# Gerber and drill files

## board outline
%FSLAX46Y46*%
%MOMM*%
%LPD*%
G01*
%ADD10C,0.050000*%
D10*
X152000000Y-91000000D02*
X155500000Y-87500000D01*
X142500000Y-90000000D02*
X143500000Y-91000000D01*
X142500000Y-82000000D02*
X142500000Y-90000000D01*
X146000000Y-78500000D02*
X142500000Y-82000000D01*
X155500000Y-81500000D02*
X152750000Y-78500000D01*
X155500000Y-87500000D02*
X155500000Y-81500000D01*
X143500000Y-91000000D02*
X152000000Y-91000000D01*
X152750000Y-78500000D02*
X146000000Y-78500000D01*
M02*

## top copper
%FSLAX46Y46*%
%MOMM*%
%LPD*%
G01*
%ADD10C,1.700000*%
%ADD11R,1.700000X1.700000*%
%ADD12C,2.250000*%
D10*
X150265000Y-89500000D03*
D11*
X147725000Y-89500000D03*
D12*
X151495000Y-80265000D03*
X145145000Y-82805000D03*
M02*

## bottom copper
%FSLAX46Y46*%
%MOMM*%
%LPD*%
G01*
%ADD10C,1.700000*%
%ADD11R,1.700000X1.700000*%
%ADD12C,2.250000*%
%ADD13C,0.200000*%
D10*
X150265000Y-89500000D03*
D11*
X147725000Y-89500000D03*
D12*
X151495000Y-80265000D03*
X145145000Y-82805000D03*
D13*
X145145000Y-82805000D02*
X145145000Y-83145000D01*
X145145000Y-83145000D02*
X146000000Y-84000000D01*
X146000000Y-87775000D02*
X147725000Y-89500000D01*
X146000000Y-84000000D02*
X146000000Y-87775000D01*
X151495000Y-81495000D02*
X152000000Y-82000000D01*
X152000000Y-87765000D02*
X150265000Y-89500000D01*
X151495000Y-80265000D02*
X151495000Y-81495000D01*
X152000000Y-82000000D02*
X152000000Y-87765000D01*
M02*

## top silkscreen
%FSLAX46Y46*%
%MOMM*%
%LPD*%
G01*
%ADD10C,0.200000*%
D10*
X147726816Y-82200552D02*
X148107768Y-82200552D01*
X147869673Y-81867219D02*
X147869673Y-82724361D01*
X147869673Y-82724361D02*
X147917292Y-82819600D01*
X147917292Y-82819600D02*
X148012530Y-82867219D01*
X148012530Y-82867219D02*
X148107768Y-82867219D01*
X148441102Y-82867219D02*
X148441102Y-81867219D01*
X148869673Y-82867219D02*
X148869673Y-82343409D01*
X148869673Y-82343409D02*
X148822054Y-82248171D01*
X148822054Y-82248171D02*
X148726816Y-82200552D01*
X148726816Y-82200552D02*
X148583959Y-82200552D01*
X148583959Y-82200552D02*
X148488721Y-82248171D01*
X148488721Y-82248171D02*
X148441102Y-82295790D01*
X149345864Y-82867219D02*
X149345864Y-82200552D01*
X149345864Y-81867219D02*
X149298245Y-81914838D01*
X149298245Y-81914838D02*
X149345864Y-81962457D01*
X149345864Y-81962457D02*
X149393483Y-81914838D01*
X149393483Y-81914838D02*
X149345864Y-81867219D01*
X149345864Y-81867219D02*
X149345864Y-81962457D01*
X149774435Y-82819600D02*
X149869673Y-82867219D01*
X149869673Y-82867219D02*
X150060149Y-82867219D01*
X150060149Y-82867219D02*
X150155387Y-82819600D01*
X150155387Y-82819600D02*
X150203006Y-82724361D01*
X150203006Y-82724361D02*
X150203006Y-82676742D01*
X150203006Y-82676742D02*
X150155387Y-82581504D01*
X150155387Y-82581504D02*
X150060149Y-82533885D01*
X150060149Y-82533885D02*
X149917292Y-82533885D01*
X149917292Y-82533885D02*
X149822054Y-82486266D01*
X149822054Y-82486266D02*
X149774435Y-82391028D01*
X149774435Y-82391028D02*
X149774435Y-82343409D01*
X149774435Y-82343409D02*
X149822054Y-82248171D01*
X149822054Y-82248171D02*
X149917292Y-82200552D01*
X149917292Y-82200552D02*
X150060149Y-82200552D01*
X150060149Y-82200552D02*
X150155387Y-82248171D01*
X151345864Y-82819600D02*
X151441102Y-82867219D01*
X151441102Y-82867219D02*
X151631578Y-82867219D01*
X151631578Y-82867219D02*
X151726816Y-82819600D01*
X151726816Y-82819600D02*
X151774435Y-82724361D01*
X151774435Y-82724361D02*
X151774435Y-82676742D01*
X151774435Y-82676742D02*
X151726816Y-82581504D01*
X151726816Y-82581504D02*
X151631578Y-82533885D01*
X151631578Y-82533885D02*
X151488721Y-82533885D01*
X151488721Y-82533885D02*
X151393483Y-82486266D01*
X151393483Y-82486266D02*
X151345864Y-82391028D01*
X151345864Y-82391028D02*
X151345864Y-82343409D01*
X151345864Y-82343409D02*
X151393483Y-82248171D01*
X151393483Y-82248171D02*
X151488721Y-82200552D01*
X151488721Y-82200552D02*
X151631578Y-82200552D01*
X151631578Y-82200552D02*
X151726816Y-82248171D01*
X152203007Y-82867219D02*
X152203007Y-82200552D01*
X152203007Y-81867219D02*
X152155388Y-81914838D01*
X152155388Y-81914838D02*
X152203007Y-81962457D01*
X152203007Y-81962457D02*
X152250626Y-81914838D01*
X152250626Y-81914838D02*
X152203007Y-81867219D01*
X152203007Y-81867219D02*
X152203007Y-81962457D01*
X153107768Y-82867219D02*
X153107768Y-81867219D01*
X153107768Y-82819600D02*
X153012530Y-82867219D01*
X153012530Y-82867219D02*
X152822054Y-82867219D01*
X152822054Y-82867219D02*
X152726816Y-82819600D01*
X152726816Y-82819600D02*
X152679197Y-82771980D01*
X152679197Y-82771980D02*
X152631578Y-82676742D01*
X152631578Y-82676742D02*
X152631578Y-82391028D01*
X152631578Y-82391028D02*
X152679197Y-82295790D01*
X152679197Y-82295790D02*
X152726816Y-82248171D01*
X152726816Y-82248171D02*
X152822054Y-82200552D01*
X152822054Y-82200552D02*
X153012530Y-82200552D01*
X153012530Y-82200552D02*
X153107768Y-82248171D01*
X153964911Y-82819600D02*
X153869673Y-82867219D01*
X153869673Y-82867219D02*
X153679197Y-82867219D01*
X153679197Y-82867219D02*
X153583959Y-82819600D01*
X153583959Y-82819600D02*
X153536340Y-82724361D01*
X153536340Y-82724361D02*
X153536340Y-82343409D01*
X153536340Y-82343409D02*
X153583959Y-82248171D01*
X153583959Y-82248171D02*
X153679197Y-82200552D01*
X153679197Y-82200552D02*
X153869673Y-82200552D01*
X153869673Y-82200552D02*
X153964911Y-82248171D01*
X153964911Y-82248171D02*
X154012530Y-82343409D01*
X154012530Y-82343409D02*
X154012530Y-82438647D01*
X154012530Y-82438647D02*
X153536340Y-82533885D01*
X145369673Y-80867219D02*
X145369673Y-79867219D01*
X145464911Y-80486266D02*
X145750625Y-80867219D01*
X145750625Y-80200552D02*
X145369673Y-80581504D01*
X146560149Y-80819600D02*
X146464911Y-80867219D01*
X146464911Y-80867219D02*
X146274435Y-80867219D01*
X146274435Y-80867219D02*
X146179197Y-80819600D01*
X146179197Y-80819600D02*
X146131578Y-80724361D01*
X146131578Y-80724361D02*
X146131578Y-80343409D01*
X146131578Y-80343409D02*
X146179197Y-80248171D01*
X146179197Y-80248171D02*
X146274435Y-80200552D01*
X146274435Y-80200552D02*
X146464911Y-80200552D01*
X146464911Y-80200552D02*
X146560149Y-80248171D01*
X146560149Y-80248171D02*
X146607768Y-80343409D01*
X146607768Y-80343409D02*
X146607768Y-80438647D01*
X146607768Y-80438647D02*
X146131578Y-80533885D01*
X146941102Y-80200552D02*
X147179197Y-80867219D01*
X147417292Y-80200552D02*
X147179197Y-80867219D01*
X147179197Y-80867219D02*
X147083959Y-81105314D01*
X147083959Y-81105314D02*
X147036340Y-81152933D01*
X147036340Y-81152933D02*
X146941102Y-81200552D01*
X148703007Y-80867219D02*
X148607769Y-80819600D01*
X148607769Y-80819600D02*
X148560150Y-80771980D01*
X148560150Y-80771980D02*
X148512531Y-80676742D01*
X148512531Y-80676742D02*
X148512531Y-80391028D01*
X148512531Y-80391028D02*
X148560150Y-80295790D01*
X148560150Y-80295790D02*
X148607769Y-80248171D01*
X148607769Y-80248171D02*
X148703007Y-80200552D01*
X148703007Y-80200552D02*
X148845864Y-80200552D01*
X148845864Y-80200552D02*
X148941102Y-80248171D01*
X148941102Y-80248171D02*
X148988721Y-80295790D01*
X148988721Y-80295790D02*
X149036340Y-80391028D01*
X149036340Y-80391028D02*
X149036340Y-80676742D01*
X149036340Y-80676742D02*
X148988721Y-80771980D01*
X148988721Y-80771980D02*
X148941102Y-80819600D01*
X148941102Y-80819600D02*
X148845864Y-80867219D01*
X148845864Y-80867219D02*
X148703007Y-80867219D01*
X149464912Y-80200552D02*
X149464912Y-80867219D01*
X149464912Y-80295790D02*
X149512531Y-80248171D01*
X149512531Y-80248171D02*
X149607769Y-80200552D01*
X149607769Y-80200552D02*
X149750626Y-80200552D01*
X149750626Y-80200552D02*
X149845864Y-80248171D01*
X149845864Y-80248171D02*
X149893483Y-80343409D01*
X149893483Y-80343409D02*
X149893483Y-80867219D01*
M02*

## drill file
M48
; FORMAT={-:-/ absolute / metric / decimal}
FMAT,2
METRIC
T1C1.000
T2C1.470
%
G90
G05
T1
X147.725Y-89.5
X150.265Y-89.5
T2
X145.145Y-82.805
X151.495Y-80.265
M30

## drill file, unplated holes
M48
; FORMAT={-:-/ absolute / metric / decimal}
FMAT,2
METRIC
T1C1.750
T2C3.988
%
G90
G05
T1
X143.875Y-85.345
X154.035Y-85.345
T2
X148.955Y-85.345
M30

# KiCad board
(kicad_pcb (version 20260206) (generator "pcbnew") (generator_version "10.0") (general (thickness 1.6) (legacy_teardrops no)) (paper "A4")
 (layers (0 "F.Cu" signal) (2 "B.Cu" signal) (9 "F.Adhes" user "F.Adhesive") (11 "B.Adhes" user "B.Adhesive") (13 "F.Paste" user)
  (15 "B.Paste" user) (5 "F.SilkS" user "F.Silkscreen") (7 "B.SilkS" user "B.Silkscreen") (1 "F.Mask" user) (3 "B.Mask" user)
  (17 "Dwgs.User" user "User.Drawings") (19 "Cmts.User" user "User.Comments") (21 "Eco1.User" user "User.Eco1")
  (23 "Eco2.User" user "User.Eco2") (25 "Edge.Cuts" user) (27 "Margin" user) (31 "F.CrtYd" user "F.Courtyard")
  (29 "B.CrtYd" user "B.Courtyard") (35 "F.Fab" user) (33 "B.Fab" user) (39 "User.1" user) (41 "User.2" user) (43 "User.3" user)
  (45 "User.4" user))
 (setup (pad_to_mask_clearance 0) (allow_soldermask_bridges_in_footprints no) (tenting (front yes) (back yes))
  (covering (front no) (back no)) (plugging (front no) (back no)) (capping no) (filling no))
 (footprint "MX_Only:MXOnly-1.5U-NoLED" (layer "F.Cu") (at 148.955 85.345)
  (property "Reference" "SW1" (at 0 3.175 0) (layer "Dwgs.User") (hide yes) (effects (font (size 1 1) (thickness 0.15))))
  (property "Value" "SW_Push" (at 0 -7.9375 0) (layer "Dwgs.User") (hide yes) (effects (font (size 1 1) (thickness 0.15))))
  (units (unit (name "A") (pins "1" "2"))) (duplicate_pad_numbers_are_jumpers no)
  (pad "" np_thru_hole circle (at -5.08 0 48.0996) (size 1.75 1.75) (drill 1.75) (layers "*.Cu" "*.Mask"))
  (pad "" np_thru_hole circle (at 0 0) (size 3.9878 3.9878) (drill 3.9878) (layers "*.Cu" "*.Mask"))
  (pad "" np_thru_hole circle (at 5.08 0 48.0996) (size 1.75 1.75) (drill 1.75) (layers "*.Cu" "*.Mask"))
  (pad "1" thru_hole circle (at -3.81 -2.54) (size 2.25 2.25) (drill 1.47) (layers "*.Cu" "B.Mask") (remove_unused_layers no)
   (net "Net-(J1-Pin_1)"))
  (pad "2" thru_hole circle (at 2.54 -5.08) (size 2.25 2.25) (drill 1.47) (layers "*.Cu" "B.Mask") (remove_unused_layers no)
   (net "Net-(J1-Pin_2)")))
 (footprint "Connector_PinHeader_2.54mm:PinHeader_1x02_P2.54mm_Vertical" (layer "B.Cu") (at 147.725 89.5 -90)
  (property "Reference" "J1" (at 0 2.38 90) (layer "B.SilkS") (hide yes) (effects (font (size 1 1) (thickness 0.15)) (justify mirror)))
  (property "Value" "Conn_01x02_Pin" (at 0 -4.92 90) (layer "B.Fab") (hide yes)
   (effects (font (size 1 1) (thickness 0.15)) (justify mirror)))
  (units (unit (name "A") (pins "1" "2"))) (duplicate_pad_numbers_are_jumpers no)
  (pad "1" thru_hole rect (at 0 0 270) (size 1.7 1.7) (drill 1) (layers "*.Cu" "*.Mask") (remove_unused_layers no) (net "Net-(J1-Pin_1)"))
  (pad "2" thru_hole circle (at 0 -2.54 270) (size 1.7 1.7) (drill 1) (layers "*.Cu" "*.Mask") (remove_unused_layers no)
   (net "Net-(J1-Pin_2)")))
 (gr_line (start 142.5 82) (end 142.5 90) (stroke (width 0.05) (type default)) (layer "Edge.Cuts"))
 (gr_line (start 142.5 90) (end 143.5 91) (stroke (width 0.05) (type default)) (layer "Edge.Cuts"))
 (gr_line (start 143.5 91) (end 152 91) (stroke (width 0.05) (type default)) (layer "Edge.Cuts"))
 (gr_line (start 146 78.5) (end 142.5 82) (stroke (width 0.05) (type default)) (layer "Edge.Cuts"))
 (gr_line (start 152 91) (end 155.5 87.5) (stroke (width 0.05) (type default)) (layer "Edge.Cuts"))
 (gr_line (start 152.75 78.5) (end 146 78.5) (stroke (width 0.05) (type default)) (layer "Edge.Cuts"))
 (gr_line (start 155.5 81.5) (end 152.75 78.5) (stroke (width 0.05) (type default)) (layer "Edge.Cuts"))
 (gr_line (start 155.5 87.5) (end 155.5 81.5) (stroke (width 0.05) (type default)) (layer "Edge.Cuts"))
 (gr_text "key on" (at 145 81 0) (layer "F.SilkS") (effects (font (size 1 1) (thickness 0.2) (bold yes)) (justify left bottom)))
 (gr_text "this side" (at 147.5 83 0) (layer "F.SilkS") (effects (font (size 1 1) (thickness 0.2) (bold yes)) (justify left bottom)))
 (segment (start 151.495 80.265) (end 151.495 81.495) (width 0.2) (layer "B.Cu") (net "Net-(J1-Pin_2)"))
 (segment (start 151.495 81.495) (end 152 82) (width 0.2) (layer "B.Cu") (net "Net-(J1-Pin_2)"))
 (segment (start 152 82) (end 152 87.765) (width 0.2) (layer "B.Cu") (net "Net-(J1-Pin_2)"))
 (segment (start 152 87.765) (end 150.265 89.5) (width 0.2) (layer "B.Cu") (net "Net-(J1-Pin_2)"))
 (segment (start 145.145 82.805) (end 145.145 83.145) (width 0.2) (layer "B.Cu") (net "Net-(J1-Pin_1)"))
 (segment (start 145.145 83.145) (end 146 84) (width 0.2) (layer "B.Cu") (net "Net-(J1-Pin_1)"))
 (segment (start 146 87.775) (end 147.725 89.5) (width 0.2) (layer "B.Cu") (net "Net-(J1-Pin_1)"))
 (segment (start 146 84) (end 146 87.775) (width 0.2) (layer "B.Cu") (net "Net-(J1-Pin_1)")))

